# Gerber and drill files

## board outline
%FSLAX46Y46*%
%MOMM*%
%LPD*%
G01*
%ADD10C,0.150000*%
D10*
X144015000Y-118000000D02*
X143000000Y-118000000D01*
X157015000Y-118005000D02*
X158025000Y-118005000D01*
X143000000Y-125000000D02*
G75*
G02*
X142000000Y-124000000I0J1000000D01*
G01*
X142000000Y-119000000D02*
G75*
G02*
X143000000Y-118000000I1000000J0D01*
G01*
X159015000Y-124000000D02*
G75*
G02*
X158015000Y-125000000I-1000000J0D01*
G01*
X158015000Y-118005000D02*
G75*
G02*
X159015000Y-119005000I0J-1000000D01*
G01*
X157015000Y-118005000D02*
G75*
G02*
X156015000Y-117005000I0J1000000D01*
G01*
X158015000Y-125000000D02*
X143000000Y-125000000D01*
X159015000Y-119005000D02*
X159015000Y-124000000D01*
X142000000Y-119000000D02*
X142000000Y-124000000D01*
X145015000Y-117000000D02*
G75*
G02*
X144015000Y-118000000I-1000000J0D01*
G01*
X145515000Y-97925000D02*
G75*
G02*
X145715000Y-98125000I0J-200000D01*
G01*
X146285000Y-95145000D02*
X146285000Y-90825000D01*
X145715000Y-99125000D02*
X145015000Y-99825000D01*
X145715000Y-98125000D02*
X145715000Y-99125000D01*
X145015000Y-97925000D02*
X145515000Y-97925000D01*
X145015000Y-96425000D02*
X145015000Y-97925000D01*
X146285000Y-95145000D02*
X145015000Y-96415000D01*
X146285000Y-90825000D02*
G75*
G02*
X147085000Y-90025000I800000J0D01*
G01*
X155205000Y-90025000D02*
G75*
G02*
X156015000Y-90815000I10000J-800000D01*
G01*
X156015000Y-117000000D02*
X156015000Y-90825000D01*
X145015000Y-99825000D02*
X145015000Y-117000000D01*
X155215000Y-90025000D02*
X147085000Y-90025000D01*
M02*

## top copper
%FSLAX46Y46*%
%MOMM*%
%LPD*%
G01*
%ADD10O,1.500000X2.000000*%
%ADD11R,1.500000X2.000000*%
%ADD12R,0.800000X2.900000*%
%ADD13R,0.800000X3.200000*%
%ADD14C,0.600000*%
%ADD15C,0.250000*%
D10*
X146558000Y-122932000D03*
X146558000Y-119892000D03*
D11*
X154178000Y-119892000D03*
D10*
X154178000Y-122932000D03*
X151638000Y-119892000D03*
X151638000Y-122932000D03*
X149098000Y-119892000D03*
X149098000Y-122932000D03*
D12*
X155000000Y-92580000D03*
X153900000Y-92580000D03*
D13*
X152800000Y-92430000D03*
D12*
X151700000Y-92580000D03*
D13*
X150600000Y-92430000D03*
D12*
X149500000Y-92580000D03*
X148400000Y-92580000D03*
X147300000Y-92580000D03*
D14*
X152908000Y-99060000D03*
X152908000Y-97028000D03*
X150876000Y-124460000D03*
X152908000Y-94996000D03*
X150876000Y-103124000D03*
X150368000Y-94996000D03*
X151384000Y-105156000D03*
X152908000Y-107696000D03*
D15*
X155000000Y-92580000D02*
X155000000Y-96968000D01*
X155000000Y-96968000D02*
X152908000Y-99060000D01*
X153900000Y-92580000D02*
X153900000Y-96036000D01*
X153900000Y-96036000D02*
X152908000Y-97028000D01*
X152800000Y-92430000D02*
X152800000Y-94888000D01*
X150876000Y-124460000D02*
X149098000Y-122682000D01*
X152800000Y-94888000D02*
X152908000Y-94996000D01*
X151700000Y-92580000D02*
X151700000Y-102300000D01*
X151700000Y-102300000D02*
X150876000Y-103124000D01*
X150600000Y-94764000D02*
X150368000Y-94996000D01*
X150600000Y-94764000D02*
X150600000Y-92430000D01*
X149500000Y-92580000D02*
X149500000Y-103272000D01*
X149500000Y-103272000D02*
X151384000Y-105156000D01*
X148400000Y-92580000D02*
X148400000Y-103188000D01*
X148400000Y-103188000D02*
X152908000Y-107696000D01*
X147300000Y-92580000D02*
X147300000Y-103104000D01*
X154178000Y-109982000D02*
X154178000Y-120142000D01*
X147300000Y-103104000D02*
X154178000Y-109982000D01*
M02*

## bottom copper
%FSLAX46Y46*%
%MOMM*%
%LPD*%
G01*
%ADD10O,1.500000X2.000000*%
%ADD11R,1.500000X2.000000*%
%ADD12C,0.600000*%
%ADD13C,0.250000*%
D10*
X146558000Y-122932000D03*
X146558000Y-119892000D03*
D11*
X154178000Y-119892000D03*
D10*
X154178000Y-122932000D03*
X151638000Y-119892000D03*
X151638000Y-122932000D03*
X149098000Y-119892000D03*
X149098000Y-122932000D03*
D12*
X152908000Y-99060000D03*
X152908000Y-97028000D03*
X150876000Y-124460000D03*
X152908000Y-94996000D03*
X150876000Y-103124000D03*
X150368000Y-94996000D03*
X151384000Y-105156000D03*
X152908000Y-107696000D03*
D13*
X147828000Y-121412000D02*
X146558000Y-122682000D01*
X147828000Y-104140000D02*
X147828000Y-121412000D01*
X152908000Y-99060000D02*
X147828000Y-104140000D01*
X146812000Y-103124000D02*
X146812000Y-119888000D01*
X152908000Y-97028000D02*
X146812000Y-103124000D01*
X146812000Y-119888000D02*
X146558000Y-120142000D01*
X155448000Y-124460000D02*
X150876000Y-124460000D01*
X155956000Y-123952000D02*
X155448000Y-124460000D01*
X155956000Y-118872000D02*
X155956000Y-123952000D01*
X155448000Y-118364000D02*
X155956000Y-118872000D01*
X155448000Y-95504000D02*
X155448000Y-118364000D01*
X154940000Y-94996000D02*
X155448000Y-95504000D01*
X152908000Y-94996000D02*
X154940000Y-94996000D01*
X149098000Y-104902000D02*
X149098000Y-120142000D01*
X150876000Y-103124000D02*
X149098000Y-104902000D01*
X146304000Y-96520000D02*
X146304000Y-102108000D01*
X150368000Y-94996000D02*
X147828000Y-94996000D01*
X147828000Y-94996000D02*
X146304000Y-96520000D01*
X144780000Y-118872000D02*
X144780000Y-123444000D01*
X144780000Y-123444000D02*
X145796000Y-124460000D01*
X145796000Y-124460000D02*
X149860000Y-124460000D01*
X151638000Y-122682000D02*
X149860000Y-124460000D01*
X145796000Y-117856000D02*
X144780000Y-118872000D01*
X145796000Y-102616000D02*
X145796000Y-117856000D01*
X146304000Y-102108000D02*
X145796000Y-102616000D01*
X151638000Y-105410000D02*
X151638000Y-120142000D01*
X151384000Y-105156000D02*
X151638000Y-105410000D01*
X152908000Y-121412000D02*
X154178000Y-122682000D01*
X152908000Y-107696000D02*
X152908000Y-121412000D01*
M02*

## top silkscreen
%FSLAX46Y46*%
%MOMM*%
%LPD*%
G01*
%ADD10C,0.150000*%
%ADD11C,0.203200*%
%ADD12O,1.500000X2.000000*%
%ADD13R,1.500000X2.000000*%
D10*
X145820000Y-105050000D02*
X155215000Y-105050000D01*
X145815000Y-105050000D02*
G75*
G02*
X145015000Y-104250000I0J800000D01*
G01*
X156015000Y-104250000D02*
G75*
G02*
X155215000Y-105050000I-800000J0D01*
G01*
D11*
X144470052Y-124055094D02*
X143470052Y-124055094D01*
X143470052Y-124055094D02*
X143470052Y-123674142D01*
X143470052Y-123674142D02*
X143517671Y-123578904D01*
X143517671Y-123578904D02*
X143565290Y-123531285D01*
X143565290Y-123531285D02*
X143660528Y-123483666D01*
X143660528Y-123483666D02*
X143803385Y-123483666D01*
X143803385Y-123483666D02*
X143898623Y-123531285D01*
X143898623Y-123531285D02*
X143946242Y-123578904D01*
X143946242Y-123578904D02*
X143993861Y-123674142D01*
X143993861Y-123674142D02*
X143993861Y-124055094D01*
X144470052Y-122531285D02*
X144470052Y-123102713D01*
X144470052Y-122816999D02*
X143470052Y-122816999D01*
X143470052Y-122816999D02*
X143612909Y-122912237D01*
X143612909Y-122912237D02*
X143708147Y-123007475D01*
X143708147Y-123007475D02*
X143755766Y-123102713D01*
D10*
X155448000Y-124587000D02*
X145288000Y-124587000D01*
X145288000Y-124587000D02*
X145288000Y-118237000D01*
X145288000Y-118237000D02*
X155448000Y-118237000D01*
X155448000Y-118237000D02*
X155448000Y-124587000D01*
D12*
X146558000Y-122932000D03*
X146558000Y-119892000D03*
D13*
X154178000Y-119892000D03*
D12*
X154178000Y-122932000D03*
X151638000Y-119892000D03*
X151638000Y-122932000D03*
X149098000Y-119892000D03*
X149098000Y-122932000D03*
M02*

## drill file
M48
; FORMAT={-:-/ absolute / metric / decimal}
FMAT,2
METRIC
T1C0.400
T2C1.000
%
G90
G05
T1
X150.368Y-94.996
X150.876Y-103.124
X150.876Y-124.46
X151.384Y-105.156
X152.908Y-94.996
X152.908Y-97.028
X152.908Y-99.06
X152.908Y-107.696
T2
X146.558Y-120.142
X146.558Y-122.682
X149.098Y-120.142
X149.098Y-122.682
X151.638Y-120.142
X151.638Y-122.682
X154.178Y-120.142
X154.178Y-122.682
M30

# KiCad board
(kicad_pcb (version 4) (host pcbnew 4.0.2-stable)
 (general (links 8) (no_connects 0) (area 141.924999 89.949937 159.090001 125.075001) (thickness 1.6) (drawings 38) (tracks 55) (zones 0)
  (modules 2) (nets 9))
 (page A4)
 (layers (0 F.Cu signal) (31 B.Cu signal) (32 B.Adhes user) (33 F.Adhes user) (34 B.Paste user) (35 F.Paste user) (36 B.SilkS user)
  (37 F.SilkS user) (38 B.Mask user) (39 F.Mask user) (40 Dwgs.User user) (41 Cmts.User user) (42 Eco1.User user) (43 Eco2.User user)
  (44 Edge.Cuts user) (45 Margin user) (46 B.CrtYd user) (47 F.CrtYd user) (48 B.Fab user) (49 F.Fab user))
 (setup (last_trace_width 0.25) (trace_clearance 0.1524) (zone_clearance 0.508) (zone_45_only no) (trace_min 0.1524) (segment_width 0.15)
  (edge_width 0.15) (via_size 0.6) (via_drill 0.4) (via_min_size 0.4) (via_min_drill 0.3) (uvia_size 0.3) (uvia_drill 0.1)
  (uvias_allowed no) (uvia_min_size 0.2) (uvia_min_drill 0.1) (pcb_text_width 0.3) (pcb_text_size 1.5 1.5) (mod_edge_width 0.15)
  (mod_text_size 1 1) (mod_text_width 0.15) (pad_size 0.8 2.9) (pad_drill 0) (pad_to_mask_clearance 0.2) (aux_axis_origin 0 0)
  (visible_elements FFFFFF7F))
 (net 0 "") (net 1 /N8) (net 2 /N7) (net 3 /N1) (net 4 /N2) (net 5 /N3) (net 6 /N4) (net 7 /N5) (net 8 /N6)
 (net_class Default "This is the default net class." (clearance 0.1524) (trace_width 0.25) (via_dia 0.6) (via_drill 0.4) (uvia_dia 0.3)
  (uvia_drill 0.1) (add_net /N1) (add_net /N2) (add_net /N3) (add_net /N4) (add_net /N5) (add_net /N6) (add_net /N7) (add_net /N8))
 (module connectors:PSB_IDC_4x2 (layer F.Cu) (at 150.368 121.412 180)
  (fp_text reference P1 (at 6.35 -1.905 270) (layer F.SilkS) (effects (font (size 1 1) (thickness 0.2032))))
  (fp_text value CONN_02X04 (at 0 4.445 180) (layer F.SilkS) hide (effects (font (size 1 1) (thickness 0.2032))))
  (fp_line (start -5.08 -3.175) (end 5.08 -3.175) (layer F.SilkS) (width 0.15))
  (fp_line (start 5.08 -3.175) (end 5.08 3.175) (layer F.SilkS) (width 0.15))
  (fp_line (start 5.08 3.175) (end -5.08 3.175) (layer F.SilkS) (width 0.15))
  (fp_line (start -5.08 3.175) (end -5.08 -3.175) (layer F.SilkS) (width 0.15))
  (pad 8 thru_hole oval (at 3.81 -1.27 180) (size 1.5 2) (drill 1 (offset 0 -0.25)) (layers *.Cu *.Mask F.SilkS) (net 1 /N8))
  (pad 7 thru_hole oval (at 3.81 1.27 180) (size 1.5 2) (drill 1 (offset 0 0.25)) (layers *.Cu *.Mask F.SilkS) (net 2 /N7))
  (pad 1 thru_hole rect (at -3.81 1.27 180) (size 1.5 2) (drill 1 (offset 0 0.25)) (layers *.Cu *.Mask F.SilkS) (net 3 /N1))
  (pad 2 thru_hole oval (at -3.81 -1.27 180) (size 1.5 2) (drill 1 (offset 0 -0.25)) (layers *.Cu *.Mask F.SilkS) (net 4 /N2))
  (pad 3 thru_hole oval (at -1.27 1.27 180) (size 1.5 2) (drill 1 (offset 0 0.25)) (layers *.Cu *.Mask F.SilkS) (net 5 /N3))
  (pad 4 thru_hole oval (at -1.27 -1.27 180) (size 1.5 2) (drill 1 (offset 0 -0.25)) (layers *.Cu *.Mask F.SilkS) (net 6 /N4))
  (pad 5 thru_hole oval (at 1.27 1.27 180) (size 1.5 2) (drill 1 (offset 0 0.25)) (layers *.Cu *.Mask F.SilkS) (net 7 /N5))
  (pad 6 thru_hole oval (at 1.27 -1.27 180) (size 1.5 2) (drill 1 (offset 0 -0.25)) (layers *.Cu *.Mask F.SilkS) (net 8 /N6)))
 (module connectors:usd (layer F.Cu) (at 147.3 92.58)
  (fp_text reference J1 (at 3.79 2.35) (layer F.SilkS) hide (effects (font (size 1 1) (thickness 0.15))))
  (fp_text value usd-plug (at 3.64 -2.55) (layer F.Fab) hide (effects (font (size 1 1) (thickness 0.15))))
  (pad 8 smd rect (at 7.7 0) (size 0.8 2.9) (layers F.Cu F.Paste F.Mask) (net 1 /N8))
  (pad 7 smd rect (at 6.6 0) (size 0.8 2.9) (layers F.Cu F.Paste F.Mask) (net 2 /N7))
  (pad 6 smd rect (at 5.5 -0.15) (size 0.8 3.2) (layers F.Cu F.Paste F.Mask) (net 8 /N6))
  (pad 5 smd rect (at 4.4 0) (size 0.8 2.9) (layers F.Cu F.Paste F.Mask) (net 7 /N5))
  (pad 4 smd rect (at 3.3 -0.15) (size 0.8 3.2) (layers F.Cu F.Paste F.Mask) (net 6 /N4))
  (pad 3 smd rect (at 2.2 0) (size 0.8 2.9) (layers F.Cu F.Paste F.Mask) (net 5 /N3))
  (pad 2 smd rect (at 1.1 0) (size 0.8 2.9) (layers F.Cu F.Paste F.Mask) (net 4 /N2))
  (pad 1 smd rect (at 0 0) (size 0.8 2.9) (layers F.Cu F.Paste F.Mask) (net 3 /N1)))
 (gr_line (start 144.015 118) (end 143 118) (angle 90) (layer Edge.Cuts) (width 0.15))
 (gr_line (start 157.015 118.005) (end 158.025 118.005) (angle 90) (layer Edge.Cuts) (width 0.15))
 (gr_arc (start 143 124) (end 143 125) (angle 90) (layer Edge.Cuts) (width 0.15))
 (gr_arc (start 143 119) (end 142 119) (angle 90) (layer Edge.Cuts) (width 0.15))
 (gr_arc (start 158.015 124) (end 159.015 124) (angle 90) (layer Edge.Cuts) (width 0.15))
 (gr_arc (start 158.015 119.005) (end 158.015 118.005) (angle 90) (layer Edge.Cuts) (width 0.15))
 (gr_arc (start 157.015 117.005) (end 157.015 118.005) (angle 90) (layer Edge.Cuts) (width 0.15))
 (gr_line (start 158.015 125) (end 143 125) (angle 90) (layer Edge.Cuts) (width 0.15))
 (gr_line (start 159.015 119.005) (end 159.015 124) (angle 90) (layer Edge.Cuts) (width 0.15))
 (gr_line (start 142 119) (end 142 124) (angle 90) (layer Edge.Cuts) (width 0.15))
 (gr_arc (start 144.015 117) (end 145.015 117) (angle 90) (layer Edge.Cuts) (width 0.15))
 (gr_line (start 145.82 105.05) (end 155.215 105.05) (angle 90) (layer F.SilkS) (width 0.15))
 (gr_arc (start 145.815 104.25) (end 145.815 105.05) (angle 90) (layer F.SilkS) (width 0.15))
 (gr_arc (start 155.215 104.25) (end 156.015 104.25) (angle 90) (layer F.SilkS) (width 0.15))
 (gr_arc (start 145.515 98.125) (end 145.715 98.125) (angle -90) (layer Edge.Cuts) (width 0.15))
 (gr_line (start 146.285 95.145) (end 146.285 90.825) (angle 90) (layer Edge.Cuts) (width 0.15))
 (gr_line (start 145.715 99.125) (end 145.015 99.825) (angle 90) (layer Edge.Cuts) (width 0.15))
 (gr_line (start 145.715 98.125) (end 145.715 99.125) (angle 90) (layer Edge.Cuts) (width 0.15))
 (gr_line (start 145.015 97.925) (end 145.515 97.925) (angle 90) (layer Edge.Cuts) (width 0.15))
 (gr_line (start 145.015 96.425) (end 145.015 97.925) (angle 90) (layer Edge.Cuts) (width 0.15))
 (gr_line (start 146.285 95.145) (end 145.015 96.415) (angle 90) (layer Edge.Cuts) (width 0.15))
 (gr_arc (start 147.085 90.825) (end 147.085 90.025) (angle -90) (layer Edge.Cuts) (width 0.15))
 (gr_arc (start 155.215 90.825) (end 156.015 90.815) (angle -90) (layer Edge.Cuts) (width 0.15))
 (gr_line (start 156.015 117) (end 156.015 90.825) (angle 90) (layer Edge.Cuts) (width 0.15))
 (gr_line (start 145.015 99.825) (end 145.015 117) (angle 90) (layer Edge.Cuts) (width 0.15))
 (gr_line (start 155.215 90.025) (end 147.085 90.025) (angle 90) (layer Edge.Cuts) (width 0.15))
 (segment (start 155 92.58) (end 155 96.968) (width 0.25) (layer F.Cu) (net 1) (status 400000))
 (segment (start 147.828 121.412) (end 146.558 122.682) (width 0.25) (layer B.Cu) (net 1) (status 800000))
 (segment (start 147.828 104.14) (end 147.828 121.412) (width 0.25) (layer B.Cu) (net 1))
 (segment (start 152.908 99.06) (end 147.828 104.14) (width 0.25) (layer B.Cu) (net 1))
 (via (at 152.908 99.06) (size 0.6) (drill 0.4) (layers F.Cu B.Cu) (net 1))
 (segment (start 155 96.968) (end 152.908 99.06) (width 0.25) (layer F.Cu) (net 1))
 (segment (start 153.9 92.58) (end 153.9 96.036) (width 0.25) (layer F.Cu) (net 2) (status 400000))
 (segment (start 146.812 103.124) (end 146.812 119.888) (width 0.25) (layer B.Cu) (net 2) (status 800000))
 (segment (start 152.908 97.028) (end 146.812 103.124) (width 0.25) (layer B.Cu) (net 2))
 (via (at 152.908 97.028) (size 0.6) (drill 0.4) (layers F.Cu B.Cu) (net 2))
 (segment (start 153.9 96.036) (end 152.908 97.028) (width 0.25) (layer F.Cu) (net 2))
 (segment (start 146.812 119.888) (end 146.558 120.142) (width 0.25) (layer B.Cu) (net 2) (status C00000))
 (segment (start 152.8 92.43) (end 152.8 94.888) (width 0.25) (layer F.Cu) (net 8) (status 400000))
 (segment (start 150.876 124.46) (end 149.098 122.682) (width 0.25) (layer F.Cu) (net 8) (status 800000))
 (via (at 150.876 124.46) (size 0.6) (drill 0.4) (layers F.Cu B.Cu) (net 8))
 (segment (start 155.448 124.46) (end 150.876 124.46) (width 0.25) (layer B.Cu) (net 8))
 (segment (start 155.956 123.952) (end 155.448 124.46) (width 0.25) (layer B.Cu) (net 8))
 (segment (start 155.956 118.872) (end 155.956 123.952) (width 0.25) (layer B.Cu) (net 8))
 (segment (start 155.448 118.364) (end 155.956 118.872) (width 0.25) (layer B.Cu) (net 8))
 (segment (start 155.448 95.504) (end 155.448 118.364) (width 0.25) (layer B.Cu) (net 8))
 (segment (start 154.94 94.996) (end 155.448 95.504) (width 0.25) (layer B.Cu) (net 8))
 (segment (start 152.908 94.996) (end 154.94 94.996) (width 0.25) (layer B.Cu) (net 8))
 (via (at 152.908 94.996) (size 0.6) (drill 0.4) (layers F.Cu B.Cu) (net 8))
 (segment (start 152.8 94.888) (end 152.908 94.996) (width 0.25) (layer F.Cu) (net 8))
 (segment (start 151.7 92.58) (end 151.7 102.3) (width 0.25) (layer F.Cu) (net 7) (status 400000))
 (segment (start 149.098 104.902) (end 149.098 120.142) (width 0.25) (layer B.Cu) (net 7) (status 800000))
 (segment (start 150.876 103.124) (end 149.098 104.902) (width 0.25) (layer B.Cu) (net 7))
 (via (at 150.876 103.124) (size 0.6) (drill 0.4) (layers F.Cu B.Cu) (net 7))
 (segment (start 151.7 102.3) (end 150.876 103.124) (width 0.25) (layer F.Cu) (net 7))
 (segment (start 146.304 96.52) (end 146.304 102.108) (width 0.25) (layer B.Cu) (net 6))
 (segment (start 150.6 94.764) (end 150.368 94.996) (width 0.25) (layer F.Cu) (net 6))
 (via (at 150.368 94.996) (size 0.6) (drill 0.4) (layers F.Cu B.Cu) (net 6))
 (segment (start 150.368 94.996) (end 147.828 94.996) (width 0.25) (layer B.Cu) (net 6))
 (segment (start 147.828 94.996) (end 146.304 96.52) (width 0.25) (layer B.Cu) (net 6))
 (segment (start 144.78 118.872) (end 144.78 123.444) (width 0.25) (layer B.Cu) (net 6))
 (segment (start 144.78 123.444) (end 145.796 124.46) (width 0.25) (layer B.Cu) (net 6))
 (segment (start 145.796 124.46) (end 149.86 124.46) (width 0.25) (layer B.Cu) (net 6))
 (segment (start 151.638 122.682) (end 149.86 124.46) (width 0.25) (layer B.Cu) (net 6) (status 400000))
 (segment (start 150.6 94.764) (end 150.6 92.43) (width 0.25) (layer F.Cu) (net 6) (status 800000))
 (segment (start 145.796 117.856) (end 144.78 118.872) (width 0.25) (layer B.Cu) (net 6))
 (segment (start 145.796 102.616) (end 145.796 117.856) (width 0.25) (layer B.Cu) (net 6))
 (segment (start 146.304 102.108) (end 145.796 102.616) (width 0.25) (layer B.Cu) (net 6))
 (segment (start 149.5 92.58) (end 149.5 103.272) (width 0.25) (layer F.Cu) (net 5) (status 400000))
 (segment (start 151.638 105.41) (end 151.638 120.142) (width 0.25) (layer B.Cu) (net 5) (status 800000))
 (segment (start 151.384 105.156) (end 151.638 105.41) (width 0.25) (layer B.Cu) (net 5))
 (via (at 151.384 105.156) (size 0.6) (drill 0.4) (layers F.Cu B.Cu) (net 5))
 (segment (start 149.5 103.272) (end 151.384 105.156) (width 0.25) (layer F.Cu) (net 5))
 (segment (start 148.4 92.58) (end 148.4 103.188) (width 0.25) (layer F.Cu) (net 4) (status 400000))
 (segment (start 152.908 121.412) (end 154.178 122.682) (width 0.25) (layer B.Cu) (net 4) (status 800000))
 (segment (start 152.908 107.696) (end 152.908 121.412) (width 0.25) (layer B.Cu) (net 4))
 (via (at 152.908 107.696) (size 0.6) (drill 0.4) (layers F.Cu B.Cu) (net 4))
 (segment (start 148.4 103.188) (end 152.908 107.696) (width 0.25) (layer F.Cu) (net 4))
 (segment (start 147.3 92.58) (end 147.3 103.104) (width 0.25) (layer F.Cu) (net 3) (status 400000))
 (segment (start 154.178 109.982) (end 154.178 120.142) (width 0.25) (layer F.Cu) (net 3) (status 800000))
 (segment (start 147.3 103.104) (end 154.178 109.982) (width 0.25) (layer F.Cu) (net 3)))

